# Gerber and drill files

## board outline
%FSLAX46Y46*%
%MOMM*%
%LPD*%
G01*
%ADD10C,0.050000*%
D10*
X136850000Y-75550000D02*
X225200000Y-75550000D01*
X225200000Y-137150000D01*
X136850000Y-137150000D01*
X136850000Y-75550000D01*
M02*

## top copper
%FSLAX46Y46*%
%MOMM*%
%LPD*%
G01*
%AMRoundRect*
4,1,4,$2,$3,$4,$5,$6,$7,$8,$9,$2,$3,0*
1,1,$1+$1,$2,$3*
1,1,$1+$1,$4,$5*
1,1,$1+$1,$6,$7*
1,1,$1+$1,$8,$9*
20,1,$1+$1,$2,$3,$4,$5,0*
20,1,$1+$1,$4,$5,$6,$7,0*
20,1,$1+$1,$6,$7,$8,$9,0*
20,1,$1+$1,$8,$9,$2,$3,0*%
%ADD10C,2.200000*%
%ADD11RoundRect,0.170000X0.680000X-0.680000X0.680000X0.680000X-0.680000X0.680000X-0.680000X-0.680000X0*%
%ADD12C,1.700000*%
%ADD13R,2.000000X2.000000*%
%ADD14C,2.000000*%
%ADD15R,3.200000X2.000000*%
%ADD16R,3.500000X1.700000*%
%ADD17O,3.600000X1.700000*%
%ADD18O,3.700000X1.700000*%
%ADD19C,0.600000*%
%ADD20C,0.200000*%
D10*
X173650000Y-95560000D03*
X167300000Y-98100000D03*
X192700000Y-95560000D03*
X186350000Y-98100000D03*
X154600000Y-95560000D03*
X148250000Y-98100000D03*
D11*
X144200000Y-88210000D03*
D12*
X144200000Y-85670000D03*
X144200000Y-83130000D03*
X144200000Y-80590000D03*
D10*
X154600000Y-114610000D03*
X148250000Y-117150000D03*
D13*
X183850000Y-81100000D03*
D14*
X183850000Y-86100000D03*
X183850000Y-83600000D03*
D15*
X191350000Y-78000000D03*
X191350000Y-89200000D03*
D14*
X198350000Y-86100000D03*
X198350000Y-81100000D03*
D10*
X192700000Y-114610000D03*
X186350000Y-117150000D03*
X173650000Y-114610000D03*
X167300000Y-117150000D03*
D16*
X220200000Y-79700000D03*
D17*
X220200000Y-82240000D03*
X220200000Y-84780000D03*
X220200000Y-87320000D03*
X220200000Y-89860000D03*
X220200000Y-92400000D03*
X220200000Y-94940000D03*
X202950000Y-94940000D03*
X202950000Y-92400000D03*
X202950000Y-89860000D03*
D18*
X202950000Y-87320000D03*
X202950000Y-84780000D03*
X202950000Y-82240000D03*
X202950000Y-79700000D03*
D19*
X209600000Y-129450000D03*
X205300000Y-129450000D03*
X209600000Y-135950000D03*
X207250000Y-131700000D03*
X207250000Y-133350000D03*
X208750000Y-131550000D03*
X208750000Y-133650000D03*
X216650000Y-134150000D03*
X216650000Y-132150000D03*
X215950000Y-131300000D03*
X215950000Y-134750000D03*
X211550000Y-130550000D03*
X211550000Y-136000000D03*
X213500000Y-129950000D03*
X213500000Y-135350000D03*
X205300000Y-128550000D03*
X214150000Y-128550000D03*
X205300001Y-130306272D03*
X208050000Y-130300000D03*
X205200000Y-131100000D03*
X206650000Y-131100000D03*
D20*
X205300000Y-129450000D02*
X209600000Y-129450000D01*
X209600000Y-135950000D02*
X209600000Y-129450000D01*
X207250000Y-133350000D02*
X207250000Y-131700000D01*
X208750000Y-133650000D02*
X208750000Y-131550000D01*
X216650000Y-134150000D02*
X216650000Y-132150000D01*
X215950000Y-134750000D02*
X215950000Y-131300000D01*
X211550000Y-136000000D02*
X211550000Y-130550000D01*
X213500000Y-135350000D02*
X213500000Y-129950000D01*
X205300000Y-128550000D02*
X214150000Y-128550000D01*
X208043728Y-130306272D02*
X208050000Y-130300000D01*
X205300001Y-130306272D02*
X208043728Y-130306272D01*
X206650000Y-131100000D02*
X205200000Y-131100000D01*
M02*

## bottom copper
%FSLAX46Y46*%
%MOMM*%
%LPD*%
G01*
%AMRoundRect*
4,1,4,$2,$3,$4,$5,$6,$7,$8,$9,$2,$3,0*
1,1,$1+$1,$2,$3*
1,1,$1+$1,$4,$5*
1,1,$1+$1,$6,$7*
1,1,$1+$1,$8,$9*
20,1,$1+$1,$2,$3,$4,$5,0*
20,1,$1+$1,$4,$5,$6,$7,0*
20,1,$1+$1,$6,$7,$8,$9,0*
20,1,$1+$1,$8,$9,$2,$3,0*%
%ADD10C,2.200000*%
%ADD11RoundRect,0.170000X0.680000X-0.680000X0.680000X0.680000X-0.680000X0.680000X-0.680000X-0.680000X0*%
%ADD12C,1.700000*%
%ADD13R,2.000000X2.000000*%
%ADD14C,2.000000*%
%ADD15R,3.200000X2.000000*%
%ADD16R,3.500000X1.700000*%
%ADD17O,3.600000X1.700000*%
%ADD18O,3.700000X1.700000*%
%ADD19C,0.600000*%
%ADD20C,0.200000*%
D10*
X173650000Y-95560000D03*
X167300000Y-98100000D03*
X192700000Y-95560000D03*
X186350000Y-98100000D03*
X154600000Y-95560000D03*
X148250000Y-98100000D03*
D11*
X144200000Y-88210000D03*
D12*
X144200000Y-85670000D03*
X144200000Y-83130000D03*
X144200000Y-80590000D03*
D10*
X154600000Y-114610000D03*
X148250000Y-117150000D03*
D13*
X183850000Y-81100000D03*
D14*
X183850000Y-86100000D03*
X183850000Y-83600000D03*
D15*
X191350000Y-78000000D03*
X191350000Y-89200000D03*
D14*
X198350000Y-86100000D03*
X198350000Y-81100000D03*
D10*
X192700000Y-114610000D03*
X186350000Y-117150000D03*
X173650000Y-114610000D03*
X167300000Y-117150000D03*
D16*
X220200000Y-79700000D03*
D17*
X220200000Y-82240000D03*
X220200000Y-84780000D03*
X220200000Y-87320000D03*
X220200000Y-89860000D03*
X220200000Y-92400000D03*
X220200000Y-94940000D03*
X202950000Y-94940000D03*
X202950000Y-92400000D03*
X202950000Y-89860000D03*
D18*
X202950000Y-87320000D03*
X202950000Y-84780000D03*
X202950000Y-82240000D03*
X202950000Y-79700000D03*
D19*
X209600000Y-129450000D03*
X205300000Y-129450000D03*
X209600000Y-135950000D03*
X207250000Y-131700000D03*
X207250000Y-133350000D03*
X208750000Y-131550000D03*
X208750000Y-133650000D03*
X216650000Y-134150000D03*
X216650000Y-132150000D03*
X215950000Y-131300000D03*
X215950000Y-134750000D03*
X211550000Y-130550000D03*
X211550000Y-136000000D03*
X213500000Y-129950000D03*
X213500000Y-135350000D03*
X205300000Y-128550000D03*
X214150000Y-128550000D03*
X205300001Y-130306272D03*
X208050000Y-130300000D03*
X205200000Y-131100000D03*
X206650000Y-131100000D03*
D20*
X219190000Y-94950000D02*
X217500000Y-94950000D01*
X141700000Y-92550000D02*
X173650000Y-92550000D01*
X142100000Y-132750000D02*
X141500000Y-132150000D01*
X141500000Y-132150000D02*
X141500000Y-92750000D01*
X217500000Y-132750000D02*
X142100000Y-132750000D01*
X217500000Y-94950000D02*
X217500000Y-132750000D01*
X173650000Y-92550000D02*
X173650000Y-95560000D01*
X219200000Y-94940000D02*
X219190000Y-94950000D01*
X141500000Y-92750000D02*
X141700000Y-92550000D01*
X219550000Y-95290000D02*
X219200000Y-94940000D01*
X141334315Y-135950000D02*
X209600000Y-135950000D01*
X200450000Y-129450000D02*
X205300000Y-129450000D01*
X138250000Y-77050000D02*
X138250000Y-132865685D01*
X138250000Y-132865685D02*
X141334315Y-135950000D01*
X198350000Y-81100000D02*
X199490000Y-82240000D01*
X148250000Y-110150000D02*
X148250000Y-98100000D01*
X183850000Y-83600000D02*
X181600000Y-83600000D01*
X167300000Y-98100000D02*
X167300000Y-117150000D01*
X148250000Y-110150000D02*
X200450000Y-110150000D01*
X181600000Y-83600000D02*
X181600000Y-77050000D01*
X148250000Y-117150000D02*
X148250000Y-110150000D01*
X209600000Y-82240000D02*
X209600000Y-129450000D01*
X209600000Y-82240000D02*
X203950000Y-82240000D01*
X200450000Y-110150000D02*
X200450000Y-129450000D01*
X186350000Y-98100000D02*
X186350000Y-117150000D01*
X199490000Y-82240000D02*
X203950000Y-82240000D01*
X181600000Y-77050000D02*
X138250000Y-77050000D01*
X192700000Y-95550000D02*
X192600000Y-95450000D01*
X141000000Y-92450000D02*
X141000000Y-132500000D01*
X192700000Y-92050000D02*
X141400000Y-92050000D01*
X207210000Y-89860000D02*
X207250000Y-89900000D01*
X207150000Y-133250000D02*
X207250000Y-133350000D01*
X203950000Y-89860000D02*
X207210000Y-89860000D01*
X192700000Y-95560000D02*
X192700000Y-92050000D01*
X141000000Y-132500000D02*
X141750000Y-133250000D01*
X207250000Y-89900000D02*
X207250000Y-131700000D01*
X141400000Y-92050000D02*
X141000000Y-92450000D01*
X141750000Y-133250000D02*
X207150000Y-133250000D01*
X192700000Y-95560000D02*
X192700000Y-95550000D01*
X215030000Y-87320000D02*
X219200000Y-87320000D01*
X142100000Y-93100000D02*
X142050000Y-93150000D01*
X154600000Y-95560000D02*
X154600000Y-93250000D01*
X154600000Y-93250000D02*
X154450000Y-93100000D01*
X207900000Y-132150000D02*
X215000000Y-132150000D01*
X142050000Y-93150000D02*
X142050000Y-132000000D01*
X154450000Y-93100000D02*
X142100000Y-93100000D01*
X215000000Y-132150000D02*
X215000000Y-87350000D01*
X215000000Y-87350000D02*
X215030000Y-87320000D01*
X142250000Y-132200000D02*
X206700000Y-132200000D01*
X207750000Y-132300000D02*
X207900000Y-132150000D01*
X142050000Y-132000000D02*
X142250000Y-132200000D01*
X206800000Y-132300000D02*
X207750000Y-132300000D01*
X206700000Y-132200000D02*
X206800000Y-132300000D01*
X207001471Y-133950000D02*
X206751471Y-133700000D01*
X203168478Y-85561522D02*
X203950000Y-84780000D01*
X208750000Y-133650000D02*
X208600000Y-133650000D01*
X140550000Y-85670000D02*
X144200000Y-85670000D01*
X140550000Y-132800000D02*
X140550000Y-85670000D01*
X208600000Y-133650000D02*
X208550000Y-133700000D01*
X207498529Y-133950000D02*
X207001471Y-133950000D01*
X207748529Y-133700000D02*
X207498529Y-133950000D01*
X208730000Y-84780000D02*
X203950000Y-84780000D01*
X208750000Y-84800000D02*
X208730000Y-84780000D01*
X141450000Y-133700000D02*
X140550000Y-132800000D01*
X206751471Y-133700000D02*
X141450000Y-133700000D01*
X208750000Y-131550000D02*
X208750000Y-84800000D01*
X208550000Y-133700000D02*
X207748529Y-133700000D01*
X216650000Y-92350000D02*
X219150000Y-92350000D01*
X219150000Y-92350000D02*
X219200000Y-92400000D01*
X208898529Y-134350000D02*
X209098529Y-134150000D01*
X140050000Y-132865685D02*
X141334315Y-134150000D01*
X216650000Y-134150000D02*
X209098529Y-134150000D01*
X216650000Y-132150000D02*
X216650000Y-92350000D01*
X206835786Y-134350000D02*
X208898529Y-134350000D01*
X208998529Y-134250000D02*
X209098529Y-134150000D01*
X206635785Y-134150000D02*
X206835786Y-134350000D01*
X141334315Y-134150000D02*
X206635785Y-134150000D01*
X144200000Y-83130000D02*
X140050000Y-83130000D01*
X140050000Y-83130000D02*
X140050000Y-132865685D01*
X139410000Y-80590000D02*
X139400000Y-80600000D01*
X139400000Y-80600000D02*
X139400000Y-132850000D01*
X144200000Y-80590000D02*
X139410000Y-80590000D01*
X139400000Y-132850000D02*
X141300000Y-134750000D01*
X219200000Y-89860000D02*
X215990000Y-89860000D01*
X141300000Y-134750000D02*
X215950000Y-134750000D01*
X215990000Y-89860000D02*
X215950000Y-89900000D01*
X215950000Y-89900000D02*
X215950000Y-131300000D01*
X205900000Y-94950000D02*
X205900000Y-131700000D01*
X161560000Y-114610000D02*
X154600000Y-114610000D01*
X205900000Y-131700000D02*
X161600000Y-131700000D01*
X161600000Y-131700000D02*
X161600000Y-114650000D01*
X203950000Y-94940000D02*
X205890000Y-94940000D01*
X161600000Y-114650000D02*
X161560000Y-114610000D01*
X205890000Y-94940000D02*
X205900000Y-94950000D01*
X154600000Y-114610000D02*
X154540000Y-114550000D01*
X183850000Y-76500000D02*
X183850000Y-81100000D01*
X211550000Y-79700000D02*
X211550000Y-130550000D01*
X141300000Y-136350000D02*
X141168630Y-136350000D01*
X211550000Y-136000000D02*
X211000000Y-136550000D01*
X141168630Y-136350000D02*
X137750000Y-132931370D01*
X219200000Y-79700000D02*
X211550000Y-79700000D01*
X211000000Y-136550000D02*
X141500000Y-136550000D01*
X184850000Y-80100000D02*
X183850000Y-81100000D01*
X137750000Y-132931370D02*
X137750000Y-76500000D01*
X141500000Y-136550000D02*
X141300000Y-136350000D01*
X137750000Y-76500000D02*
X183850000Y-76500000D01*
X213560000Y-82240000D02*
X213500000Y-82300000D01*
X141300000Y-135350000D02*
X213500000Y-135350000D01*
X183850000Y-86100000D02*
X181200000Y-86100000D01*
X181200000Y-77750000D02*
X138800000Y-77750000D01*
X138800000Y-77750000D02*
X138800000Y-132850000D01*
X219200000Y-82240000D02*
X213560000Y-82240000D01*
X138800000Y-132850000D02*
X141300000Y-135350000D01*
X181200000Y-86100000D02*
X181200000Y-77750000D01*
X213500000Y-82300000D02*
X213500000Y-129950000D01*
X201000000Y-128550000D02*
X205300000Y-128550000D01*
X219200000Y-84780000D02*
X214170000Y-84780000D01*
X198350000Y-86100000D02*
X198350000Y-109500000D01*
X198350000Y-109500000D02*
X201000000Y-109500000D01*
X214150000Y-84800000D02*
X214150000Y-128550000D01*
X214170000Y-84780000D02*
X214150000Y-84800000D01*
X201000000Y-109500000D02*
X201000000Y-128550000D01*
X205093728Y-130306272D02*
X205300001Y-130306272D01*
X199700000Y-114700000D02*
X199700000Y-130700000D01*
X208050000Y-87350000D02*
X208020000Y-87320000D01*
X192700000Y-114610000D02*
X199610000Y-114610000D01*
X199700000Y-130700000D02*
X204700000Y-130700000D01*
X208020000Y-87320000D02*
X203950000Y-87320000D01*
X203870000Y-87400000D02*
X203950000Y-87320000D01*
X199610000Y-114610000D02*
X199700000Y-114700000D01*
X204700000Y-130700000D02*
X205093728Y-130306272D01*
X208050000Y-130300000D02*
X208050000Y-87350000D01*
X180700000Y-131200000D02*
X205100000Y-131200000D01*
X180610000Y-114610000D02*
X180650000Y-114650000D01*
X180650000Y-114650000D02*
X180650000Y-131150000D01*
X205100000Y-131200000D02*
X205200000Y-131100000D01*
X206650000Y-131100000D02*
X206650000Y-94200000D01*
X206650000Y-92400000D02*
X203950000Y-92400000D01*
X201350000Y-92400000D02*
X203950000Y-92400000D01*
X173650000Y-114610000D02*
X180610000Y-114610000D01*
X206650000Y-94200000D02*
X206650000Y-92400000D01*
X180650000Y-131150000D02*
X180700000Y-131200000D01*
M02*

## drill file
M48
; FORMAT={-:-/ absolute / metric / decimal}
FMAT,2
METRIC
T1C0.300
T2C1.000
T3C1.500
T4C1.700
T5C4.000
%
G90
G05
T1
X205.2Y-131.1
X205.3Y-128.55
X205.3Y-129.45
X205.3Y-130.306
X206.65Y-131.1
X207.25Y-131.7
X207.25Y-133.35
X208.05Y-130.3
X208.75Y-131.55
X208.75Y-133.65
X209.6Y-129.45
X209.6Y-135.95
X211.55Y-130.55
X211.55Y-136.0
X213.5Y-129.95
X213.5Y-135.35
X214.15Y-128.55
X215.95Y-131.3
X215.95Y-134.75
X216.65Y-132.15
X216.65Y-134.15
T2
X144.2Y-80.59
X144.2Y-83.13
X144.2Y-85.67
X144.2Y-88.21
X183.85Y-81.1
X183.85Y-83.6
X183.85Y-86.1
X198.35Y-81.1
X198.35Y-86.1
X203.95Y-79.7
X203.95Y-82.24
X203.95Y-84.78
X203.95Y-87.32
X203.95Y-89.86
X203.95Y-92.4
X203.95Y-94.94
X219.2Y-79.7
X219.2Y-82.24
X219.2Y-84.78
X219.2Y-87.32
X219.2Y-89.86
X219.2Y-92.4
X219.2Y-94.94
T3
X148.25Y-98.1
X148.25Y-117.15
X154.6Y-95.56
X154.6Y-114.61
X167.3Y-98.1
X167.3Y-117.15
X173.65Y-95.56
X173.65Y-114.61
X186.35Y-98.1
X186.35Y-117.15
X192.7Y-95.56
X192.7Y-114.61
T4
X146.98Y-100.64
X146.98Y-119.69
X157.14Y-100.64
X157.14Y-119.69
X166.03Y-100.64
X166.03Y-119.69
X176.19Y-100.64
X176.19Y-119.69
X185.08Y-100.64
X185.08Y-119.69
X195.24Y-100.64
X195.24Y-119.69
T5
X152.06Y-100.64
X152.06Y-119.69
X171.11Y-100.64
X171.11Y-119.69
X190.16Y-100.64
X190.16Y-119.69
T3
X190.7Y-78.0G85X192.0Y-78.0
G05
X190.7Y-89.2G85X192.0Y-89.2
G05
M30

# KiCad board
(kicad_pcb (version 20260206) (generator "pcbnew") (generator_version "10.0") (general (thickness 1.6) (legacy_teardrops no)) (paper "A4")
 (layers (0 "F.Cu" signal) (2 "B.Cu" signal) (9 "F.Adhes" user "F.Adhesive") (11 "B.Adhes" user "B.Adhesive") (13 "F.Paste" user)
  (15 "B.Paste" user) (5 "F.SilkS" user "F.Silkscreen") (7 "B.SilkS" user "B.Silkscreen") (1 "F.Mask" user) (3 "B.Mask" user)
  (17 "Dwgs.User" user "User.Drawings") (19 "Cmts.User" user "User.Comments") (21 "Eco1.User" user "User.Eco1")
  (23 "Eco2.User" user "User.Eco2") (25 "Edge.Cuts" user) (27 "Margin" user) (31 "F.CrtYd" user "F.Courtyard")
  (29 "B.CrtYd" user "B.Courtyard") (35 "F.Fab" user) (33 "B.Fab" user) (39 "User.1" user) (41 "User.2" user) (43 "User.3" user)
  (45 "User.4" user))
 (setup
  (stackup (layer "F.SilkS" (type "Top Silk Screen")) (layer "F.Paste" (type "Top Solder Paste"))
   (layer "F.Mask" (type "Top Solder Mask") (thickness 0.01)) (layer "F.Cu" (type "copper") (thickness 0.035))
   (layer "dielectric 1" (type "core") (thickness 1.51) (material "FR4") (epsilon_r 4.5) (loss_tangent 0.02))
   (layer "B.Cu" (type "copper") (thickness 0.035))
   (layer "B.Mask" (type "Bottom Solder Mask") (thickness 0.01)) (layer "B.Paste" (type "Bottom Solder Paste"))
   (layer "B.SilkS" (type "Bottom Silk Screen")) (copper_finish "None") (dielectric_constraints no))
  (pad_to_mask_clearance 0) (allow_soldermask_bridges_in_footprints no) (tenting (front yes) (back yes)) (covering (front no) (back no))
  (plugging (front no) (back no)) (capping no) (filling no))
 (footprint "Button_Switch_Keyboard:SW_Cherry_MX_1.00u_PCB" (layer "F.Cu") (at 173.65 95.56)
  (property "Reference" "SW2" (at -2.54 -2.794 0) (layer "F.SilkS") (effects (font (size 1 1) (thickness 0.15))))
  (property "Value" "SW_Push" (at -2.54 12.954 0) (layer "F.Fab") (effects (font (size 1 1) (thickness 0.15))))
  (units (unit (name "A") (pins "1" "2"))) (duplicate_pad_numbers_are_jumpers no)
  (pad "" np_thru_hole circle (at -7.62 5.08) (size 1.7 1.7) (drill 1.7) (layers "*.Cu" "*.Mask"))
  (pad "" np_thru_hole circle (at -2.54 5.08) (size 4 4) (drill 4) (layers "*.Cu" "*.Mask"))
  (pad "" np_thru_hole circle (at 2.54 5.08) (size 1.7 1.7) (drill 1.7) (layers "*.Cu" "*.Mask"))
  (pad "1" thru_hole circle (at 0 0) (size 2.2 2.2) (drill 1.5) (layers "*.Cu" "*.Mask") (remove_unused_layers no)
   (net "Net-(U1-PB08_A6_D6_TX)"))
  (pad "2" thru_hole circle (at -6.35 2.54) (size 2.2 2.2) (drill 1.5) (layers "*.Cu" "*.Mask") (remove_unused_layers no) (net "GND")))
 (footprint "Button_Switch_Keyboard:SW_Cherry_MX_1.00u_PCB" (layer "F.Cu") (at 192.7 95.56)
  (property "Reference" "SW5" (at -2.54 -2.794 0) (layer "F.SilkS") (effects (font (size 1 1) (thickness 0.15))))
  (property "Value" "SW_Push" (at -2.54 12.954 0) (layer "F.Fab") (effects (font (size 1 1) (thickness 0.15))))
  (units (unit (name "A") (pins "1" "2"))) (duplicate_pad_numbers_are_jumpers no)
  (pad "" np_thru_hole circle (at -7.62 5.08) (size 1.7 1.7) (drill 1.7) (layers "*.Cu" "*.Mask"))
  (pad "" np_thru_hole circle (at -2.54 5.08) (size 4 4) (drill 4) (layers "*.Cu" "*.Mask"))
  (pad "" np_thru_hole circle (at 2.54 5.08) (size 1.7 1.7) (drill 1.7) (layers "*.Cu" "*.Mask"))
  (pad "1" thru_hole circle (at 0 0) (size 2.2 2.2) (drill 1.5) (layers "*.Cu" "*.Mask") (remove_unused_layers no)
   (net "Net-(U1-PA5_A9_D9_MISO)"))
  (pad "2" thru_hole circle (at -6.35 2.54) (size 2.2 2.2) (drill 1.5) (layers "*.Cu" "*.Mask") (remove_unused_layers no) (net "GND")))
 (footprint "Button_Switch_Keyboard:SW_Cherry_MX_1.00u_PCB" (layer "F.Cu") (at 154.6 95.56)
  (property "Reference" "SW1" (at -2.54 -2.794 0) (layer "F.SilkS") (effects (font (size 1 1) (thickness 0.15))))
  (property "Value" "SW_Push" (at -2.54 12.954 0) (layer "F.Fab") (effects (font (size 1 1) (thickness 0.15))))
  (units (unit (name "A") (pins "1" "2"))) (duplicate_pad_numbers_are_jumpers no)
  (pad "" np_thru_hole circle (at -7.62 5.08) (size 1.7 1.7) (drill 1.7) (layers "*.Cu" "*.Mask"))
  (pad "" np_thru_hole circle (at -2.54 5.08) (size 4 4) (drill 4) (layers "*.Cu" "*.Mask"))
  (pad "" np_thru_hole circle (at 2.54 5.08) (size 1.7 1.7) (drill 1.7) (layers "*.Cu" "*.Mask"))
  (pad "1" thru_hole circle (at 0 0) (size 2.2 2.2) (drill 1.5) (layers "*.Cu" "*.Mask") (remove_unused_layers no)
   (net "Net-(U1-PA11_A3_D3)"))
  (pad "2" thru_hole circle (at -6.35 2.54) (size 2.2 2.2) (drill 1.5) (layers "*.Cu" "*.Mask") (remove_unused_layers no) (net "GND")))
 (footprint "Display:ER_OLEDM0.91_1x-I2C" (layer "F.Cu") (at 144.2 88.21 90)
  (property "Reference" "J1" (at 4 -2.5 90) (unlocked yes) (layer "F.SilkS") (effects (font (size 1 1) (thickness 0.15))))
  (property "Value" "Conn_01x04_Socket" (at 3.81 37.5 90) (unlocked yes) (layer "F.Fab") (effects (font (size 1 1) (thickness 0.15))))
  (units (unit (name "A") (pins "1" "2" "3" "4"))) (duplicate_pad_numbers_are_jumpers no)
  (pad "1" thru_hole roundrect (at 0 0 90) (size 1.7 1.7) (drill 1) (layers "*.Cu" "*.Mask") (remove_unused_layers no)
   (roundrect_rratio 0.1) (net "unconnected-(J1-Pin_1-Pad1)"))
  (pad "2" thru_hole circle (at 2.54 0 90) (size 1.7 1.7) (drill 1) (layers "*.Cu" "*.Mask") (remove_unused_layers no)
   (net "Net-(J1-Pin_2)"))
  (pad "3" thru_hole circle (at 5.08 0 90) (size 1.7 1.7) (drill 1) (layers "*.Cu" "*.Mask") (remove_unused_layers no)
   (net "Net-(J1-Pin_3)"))
  (pad "4" thru_hole circle (at 7.62 0 90) (size 1.7 1.7) (drill 1) (layers "*.Cu" "*.Mask") (remove_unused_layers no)
   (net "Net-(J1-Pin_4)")))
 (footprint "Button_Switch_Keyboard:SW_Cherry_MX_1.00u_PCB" (layer "F.Cu") (at 154.6 114.61)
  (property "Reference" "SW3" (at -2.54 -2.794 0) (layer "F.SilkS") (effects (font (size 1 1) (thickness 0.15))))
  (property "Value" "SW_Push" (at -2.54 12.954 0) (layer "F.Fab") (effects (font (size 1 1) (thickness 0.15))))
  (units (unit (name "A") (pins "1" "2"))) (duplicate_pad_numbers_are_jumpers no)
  (pad "" np_thru_hole circle (at -7.62 5.08) (size 1.7 1.7) (drill 1.7) (layers "*.Cu" "*.Mask"))
  (pad "" np_thru_hole circle (at -2.54 5.08) (size 4 4) (drill 4) (layers "*.Cu" "*.Mask"))
  (pad "" np_thru_hole circle (at 2.54 5.08) (size 1.7 1.7) (drill 1.7) (layers "*.Cu" "*.Mask"))
  (pad "1" thru_hole circle (at 0 0) (size 2.2 2.2) (drill 1.5) (layers "*.Cu" "*.Mask") (remove_unused_layers no)
   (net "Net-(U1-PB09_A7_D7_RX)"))
  (pad "2" thru_hole circle (at -6.35 2.54) (size 2.2 2.2) (drill 1.5) (layers "*.Cu" "*.Mask") (remove_unused_layers no) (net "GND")))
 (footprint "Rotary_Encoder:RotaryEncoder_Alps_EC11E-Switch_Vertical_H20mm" (layer "F.Cu") (at 183.85 81.1)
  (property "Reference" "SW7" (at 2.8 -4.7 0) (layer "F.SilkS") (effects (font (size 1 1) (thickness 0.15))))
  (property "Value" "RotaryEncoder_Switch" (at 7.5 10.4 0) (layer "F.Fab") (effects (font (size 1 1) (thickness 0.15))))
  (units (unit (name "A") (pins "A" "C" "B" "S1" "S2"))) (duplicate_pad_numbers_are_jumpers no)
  (pad "A" thru_hole rect (at 0 0) (size 2 2) (drill 1) (layers "*.Cu" "*.Mask") (remove_unused_layers no) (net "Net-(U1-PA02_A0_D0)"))
  (pad "B" thru_hole circle (at 0 5) (size 2 2) (drill 1) (layers "*.Cu" "*.Mask") (remove_unused_layers no) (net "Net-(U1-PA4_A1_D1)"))
  (pad "C" thru_hole circle (at 0 2.5) (size 2 2) (drill 1) (layers "*.Cu" "*.Mask") (remove_unused_layers no) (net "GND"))
  (pad "MP" thru_hole rect (at 7.5 -3.1) (size 3.2 2) (drill oval 2.8 1.5) (layers "*.Cu" "*.Mask") (remove_unused_layers no))
  (pad "MP" thru_hole rect (at 7.5 8.1) (size 3.2 2) (drill oval 2.8 1.5) (layers "*.Cu" "*.Mask") (remove_unused_layers no))
  (pad "S1" thru_hole circle (at 14.5 5) (size 2 2) (drill 1) (layers "*.Cu" "*.Mask") (remove_unused_layers no) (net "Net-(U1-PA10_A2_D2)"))
  (pad "S2" thru_hole circle (at 14.5 0) (size 2 2) (drill 1) (layers "*.Cu" "*.Mask") (remove_unused_layers no) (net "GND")))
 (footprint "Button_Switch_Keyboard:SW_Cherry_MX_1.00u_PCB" (layer "F.Cu") (at 192.7 114.61)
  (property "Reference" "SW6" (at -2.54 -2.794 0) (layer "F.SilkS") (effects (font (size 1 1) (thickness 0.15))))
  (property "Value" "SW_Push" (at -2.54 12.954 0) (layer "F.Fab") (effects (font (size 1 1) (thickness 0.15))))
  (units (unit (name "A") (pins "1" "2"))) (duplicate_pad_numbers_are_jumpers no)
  (pad "" np_thru_hole circle (at -7.62 5.08) (size 1.7 1.7) (drill 1.7) (layers "*.Cu" "*.Mask"))
  (pad "" np_thru_hole circle (at -2.54 5.08) (size 4 4) (drill 4) (layers "*.Cu" "*.Mask"))
  (pad "" np_thru_hole circle (at 2.54 5.08) (size 1.7 1.7) (drill 1.7) (layers "*.Cu" "*.Mask"))
  (pad "1" thru_hole circle (at 0 0) (size 2.2 2.2) (drill 1.5) (layers "*.Cu" "*.Mask") (remove_unused_layers no)
   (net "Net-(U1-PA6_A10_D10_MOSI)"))
  (pad "2" thru_hole circle (at -6.35 2.54) (size 2.2 2.2) (drill 1.5) (layers "*.Cu" "*.Mask") (remove_unused_layers no) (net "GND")))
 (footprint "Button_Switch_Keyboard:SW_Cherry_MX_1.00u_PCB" (layer "F.Cu") (at 173.65 114.61)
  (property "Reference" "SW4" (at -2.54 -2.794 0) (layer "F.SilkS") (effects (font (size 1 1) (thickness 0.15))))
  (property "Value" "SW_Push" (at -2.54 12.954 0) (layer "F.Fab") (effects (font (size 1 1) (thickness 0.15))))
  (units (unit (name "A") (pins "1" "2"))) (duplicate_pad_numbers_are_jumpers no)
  (pad "" np_thru_hole circle (at -7.62 5.08) (size 1.7 1.7) (drill 1.7) (layers "*.Cu" "*.Mask"))
  (pad "" np_thru_hole circle (at -2.54 5.08) (size 4 4) (drill 4) (layers "*.Cu" "*.Mask"))
  (pad "" np_thru_hole circle (at 2.54 5.08) (size 1.7 1.7) (drill 1.7) (layers "*.Cu" "*.Mask"))
  (pad "1" thru_hole circle (at 0 0) (size 2.2 2.2) (drill 1.5) (layers "*.Cu" "*.Mask") (remove_unused_layers no)
   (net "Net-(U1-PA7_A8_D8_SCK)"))
  (pad "2" thru_hole circle (at -6.35 2.54) (size 2.2 2.2) (drill 1.5) (layers "*.Cu" "*.Mask") (remove_unused_layers no) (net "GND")))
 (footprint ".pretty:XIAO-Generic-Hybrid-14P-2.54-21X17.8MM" (layer "B.Cu") (at 211.575 87.32 180)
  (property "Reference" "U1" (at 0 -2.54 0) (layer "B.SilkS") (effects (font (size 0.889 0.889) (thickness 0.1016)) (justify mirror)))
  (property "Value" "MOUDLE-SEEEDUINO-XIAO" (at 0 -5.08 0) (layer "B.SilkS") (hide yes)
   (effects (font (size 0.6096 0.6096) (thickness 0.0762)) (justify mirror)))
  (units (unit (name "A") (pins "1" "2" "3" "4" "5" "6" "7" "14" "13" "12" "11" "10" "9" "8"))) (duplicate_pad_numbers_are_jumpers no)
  (pad "1" thru_hole rect (at -7.625 7.62 180) (size 3.5 1.7) (drill 1 (offset -1 0)) (layers "*.Cu" "*.Mask") (remove_unused_layers no)
   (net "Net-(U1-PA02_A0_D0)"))
  (pad "2" thru_hole oval (at -7.625 5.08 180) (size 3.6 1.7) (drill 1 (offset -1 0)) (layers "*.Cu" "*.Mask") (remove_unused_layers no)
   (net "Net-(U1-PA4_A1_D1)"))
  (pad "3" thru_hole oval (at -7.625 2.54 180) (size 3.6 1.7) (drill 1 (offset -1 0)) (layers "*.Cu" "*.Mask") (remove_unused_layers no)
   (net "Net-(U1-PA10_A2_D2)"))
  (pad "4" thru_hole oval (at -7.625 0 180) (size 3.6 1.7) (drill 1 (offset -1 0)) (layers "*.Cu" "*.Mask") (remove_unused_layers no)
   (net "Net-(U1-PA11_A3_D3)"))
  (pad "5" thru_hole oval (at -7.625 -2.54 180) (size 3.6 1.7) (drill 1 (offset -1 0)) (layers "*.Cu" "*.Mask") (remove_unused_layers no)
   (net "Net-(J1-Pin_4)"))
  (pad "6" thru_hole oval (at -7.625 -5.08) (size 3.6 1.7) (drill 1 (offset 1 0)) (layers "*.Cu" "*.Mask") (remove_unused_layers no)
   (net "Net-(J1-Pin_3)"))
  (pad "7" thru_hole oval (at -7.625 -7.62 180) (size 3.6 1.7) (drill 1 (offset -1 0)) (layers "*.Cu" "*.Mask") (remove_unused_layers no)
   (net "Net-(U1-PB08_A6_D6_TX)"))
  (pad "8" thru_hole oval (at 7.625 -7.62 180) (size 3.6 1.7) (drill 1 (offset 1 0)) (layers "*.Cu" "*.Mask") (remove_unused_layers no)
   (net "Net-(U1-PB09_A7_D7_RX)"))
  (pad "9" thru_hole oval (at 7.625 -5.08 180) (size 3.6 1.7) (drill 1 (offset 1 0)) (layers "*.Cu" "*.Mask") (remove_unused_layers no)
   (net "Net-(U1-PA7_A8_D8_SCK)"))
  (pad "10" thru_hole oval (at 7.625 -2.54 180) (size 3.6 1.7) (drill 1 (offset 1 0)) (layers "*.Cu" "*.Mask") (remove_unused_layers no)
   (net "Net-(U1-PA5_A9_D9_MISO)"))
  (pad "11" thru_hole oval (at 7.625 0 180) (size 3.7 1.7) (drill 1 (offset 1 0)) (layers "*.Cu" "*.Mask") (remove_unused_layers no)
   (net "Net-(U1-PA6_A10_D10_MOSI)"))
  (pad "12" thru_hole oval (at 7.625 2.54 180) (size 3.7 1.7) (drill 1 (offset 1 0)) (layers "*.Cu" "*.Mask") (remove_unused_layers no)
   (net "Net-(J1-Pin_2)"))
  (pad "13" thru_hole oval (at 7.625 5.08 180) (size 3.7 1.7) (drill 1 (offset 1 0)) (layers "*.Cu" "*.Mask") (remove_unused_layers no)
   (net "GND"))
  (pad "14" thru_hole oval (at 7.625 7.62 180) (size 3.7 1.7) (drill 1 (offset 1 0)) (layers "*.Cu" "*.Mask") (remove_unused_layers no)
   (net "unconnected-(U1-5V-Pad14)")))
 (gr_rect (start 136.85 75.55) (end 225.2 137.15) (stroke (width 0.05) (type default)) (fill no) (layer "Edge.Cuts"))
 (segment (start 219.19 94.95) (end 217.5 94.95) (width 0.2) (layer "B.Cu") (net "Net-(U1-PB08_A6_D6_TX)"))
 (segment (start 141.7 92.55) (end 173.65 92.55) (width 0.2) (layer "B.Cu") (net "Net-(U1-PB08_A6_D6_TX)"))
 (segment (start 142.1 132.75) (end 141.5 132.15) (width 0.2) (layer "B.Cu") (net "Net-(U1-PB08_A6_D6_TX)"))
 (segment (start 141.5 132.15) (end 141.5 92.75) (width 0.2) (layer "B.Cu") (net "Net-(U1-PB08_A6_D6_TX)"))
 (segment (start 217.5 132.75) (end 142.1 132.75) (width 0.2) (layer "B.Cu") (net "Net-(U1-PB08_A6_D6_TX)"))
 (segment (start 217.5 94.95) (end 217.5 132.75) (width 0.2) (layer "B.Cu") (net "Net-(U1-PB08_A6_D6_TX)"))
 (segment (start 173.65 92.55) (end 173.65 95.56) (width 0.2) (layer "B.Cu") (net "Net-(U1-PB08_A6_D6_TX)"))
 (segment (start 219.2 94.94) (end 219.19 94.95) (width 0.2) (layer "B.Cu") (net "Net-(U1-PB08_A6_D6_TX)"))
 (segment (start 141.5 92.75) (end 141.7 92.55) (width 0.2) (layer "B.Cu") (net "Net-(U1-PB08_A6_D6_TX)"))
 (segment (start 219.55 95.29) (end 219.2 94.94) (width 0.2) (layer "B.Cu") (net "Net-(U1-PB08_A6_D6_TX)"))
 (segment (start 205.3 129.45) (end 209.6 129.45) (width 0.2) (layer "F.Cu") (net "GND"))
 (segment (start 209.6 135.95) (end 209.6 129.45) (width 0.2) (layer "F.Cu") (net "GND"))
 (via (at 209.6 129.45) (size 0.6) (drill 0.3) (layers "F.Cu" "B.Cu") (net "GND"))
 (via (at 205.3 129.45) (size 0.6) (drill 0.3) (layers "F.Cu" "B.Cu") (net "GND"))
 (via (at 209.6 135.95) (size 0.6) (drill 0.3) (layers "F.Cu" "B.Cu") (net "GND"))
 (segment (start 141.334315 135.95) (end 209.6 135.95) (width 0.2) (layer "B.Cu") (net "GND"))
 (segment (start 200.45 129.45) (end 205.3 129.45) (width 0.2) (layer "B.Cu") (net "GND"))
 (segment (start 138.25 77.05) (end 138.25 132.865685) (width 0.2) (layer "B.Cu") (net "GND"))
 (segment (start 138.25 132.865685) (end 141.334315 135.95) (width 0.2) (layer "B.Cu") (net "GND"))
 (segment (start 198.35 81.1) (end 199.49 82.24) (width 0.2) (layer "B.Cu") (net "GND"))
 (segment (start 148.25 110.15) (end 148.25 98.1) (width 0.2) (layer "B.Cu") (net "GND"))
 (segment (start 183.85 83.6) (end 181.6 83.6) (width 0.2) (layer "B.Cu") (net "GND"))
 (segment (start 167.3 98.1) (end 167.3 117.15) (width 0.2) (layer "B.Cu") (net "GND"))
 (segment (start 148.25 110.15) (end 200.45 110.15) (width 0.2) (layer "B.Cu") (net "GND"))
 (segment (start 181.6 83.6) (end 181.6 77.05) (width 0.2) (layer "B.Cu") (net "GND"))
 (segment (start 148.25 117.15) (end 148.25 110.15) (width 0.2) (layer "B.Cu") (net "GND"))
 (segment (start 209.6 82.24) (end 209.6 129.45) (width 0.2) (layer "B.Cu") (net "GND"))
 (segment (start 209.6 82.24) (end 203.95 82.24) (width 0.2) (layer "B.Cu") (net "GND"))
 (segment (start 200.45 110.15) (end 200.45 129.45) (width 0.2) (layer "B.Cu") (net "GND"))
 (segment (start 186.35 98.1) (end 186.35 117.15) (width 0.2) (layer "B.Cu") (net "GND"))
 (segment (start 199.49 82.24) (end 203.95 82.24) (width 0.2) (layer "B.Cu") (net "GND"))
 (segment (start 181.6 77.05) (end 138.25 77.05) (width 0.2) (layer "B.Cu") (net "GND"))
 (segment (start 207.25 133.35) (end 207.25 131.7) (width 0.2) (layer "F.Cu") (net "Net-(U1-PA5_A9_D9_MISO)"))
 (via (at 207.25 131.7) (size 0.6) (drill 0.3) (layers "F.Cu" "B.Cu") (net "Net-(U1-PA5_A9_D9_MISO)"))
 (via (at 207.25 133.35) (size 0.6) (drill 0.3) (layers "F.Cu" "B.Cu") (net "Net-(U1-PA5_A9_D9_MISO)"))
 (segment (start 192.7 95.55) (end 192.6 95.45) (width 0.2) (layer "B.Cu") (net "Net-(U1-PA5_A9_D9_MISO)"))
 (segment (start 141 92.45) (end 141 132.5) (width 0.2) (layer "B.Cu") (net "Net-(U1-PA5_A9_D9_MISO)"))
 (segment (start 192.7 92.05) (end 141.4 92.05) (width 0.2) (layer "B.Cu") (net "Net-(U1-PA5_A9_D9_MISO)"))
 (segment (start 207.21 89.86) (end 207.25 89.9) (width 0.2) (layer "B.Cu") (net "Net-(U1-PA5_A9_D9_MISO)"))
 (segment (start 207.15 133.25) (end 207.25 133.35) (width 0.2) (layer "B.Cu") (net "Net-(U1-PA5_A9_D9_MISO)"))
 (segment (start 203.95 89.86) (end 207.21 89.86) (width 0.2) (layer "B.Cu") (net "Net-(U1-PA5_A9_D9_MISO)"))
 (segment (start 192.7 95.56) (end 192.7 92.05) (width 0.2) (layer "B.Cu") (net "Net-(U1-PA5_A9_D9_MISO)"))
 (segment (start 141 132.5) (end 141.75 133.25) (width 0.2) (layer "B.Cu") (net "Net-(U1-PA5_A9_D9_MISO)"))
 (segment (start 207.25 89.9) (end 207.25 131.7) (width 0.2) (layer "B.Cu") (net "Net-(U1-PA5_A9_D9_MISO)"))
 (segment (start 141.4 92.05) (end 141 92.45) (width 0.2) (layer "B.Cu") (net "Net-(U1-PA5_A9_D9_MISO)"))
 (segment (start 141.75 133.25) (end 207.15 133.25) (width 0.2) (layer "B.Cu") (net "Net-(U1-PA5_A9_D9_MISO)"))
 (segment (start 192.7 95.56) (end 192.7 95.55) (width 0.2) (layer "B.Cu") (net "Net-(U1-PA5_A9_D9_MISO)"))
 (segment (start 215.03 87.32) (end 219.2 87.32) (width 0.2) (layer "B.Cu") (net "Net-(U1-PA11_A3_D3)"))
 (segment (start 142.1 93.1) (end 142.05 93.15) (width 0.2) (layer "B.Cu") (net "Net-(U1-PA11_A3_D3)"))
 (segment (start 154.6 95.56) (end 154.6 93.25) (width 0.2) (layer "B.Cu") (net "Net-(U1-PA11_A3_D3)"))
 (segment (start 154.6 93.25) (end 154.45 93.1) (width 0.2) (layer "B.Cu") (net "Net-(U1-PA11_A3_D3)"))
 (segment (start 207.9 132.15) (end 215 132.15) (width 0.2) (layer "B.Cu") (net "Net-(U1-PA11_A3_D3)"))
 (segment (start 142.05 93.15) (end 142.05 132) (width 0.2) (layer "B.Cu") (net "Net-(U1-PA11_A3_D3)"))
 (segment (start 154.45 93.1) (end 142.1 93.1) (width 0.2) (layer "B.Cu") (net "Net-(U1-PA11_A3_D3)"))
 (segment (start 215 132.15) (end 215 87.35) (width 0.2) (layer "B.Cu") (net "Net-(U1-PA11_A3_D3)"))
 (segment (start 215 87.35) (end 215.03 87.32) (width 0.2) (layer "B.Cu") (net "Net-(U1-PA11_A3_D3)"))
 (segment (start 142.25 132.2) (end 206.7 132.2) (width 0.2) (layer "B.Cu") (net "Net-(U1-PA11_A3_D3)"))
 (segment (start 207.75 132.3) (end 207.9 132.15) (width 0.2) (layer "B.Cu") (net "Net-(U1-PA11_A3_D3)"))
 (segment (start 142.05 132) (end 142.25 132.2) (width 0.2) (layer "B.Cu") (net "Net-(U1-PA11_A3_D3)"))
 (segment (start 206.8 132.3) (end 207.75 132.3) (width 0.2) (layer "B.Cu") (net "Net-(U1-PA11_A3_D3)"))
 (segment (start 206.7 132.2) (end 206.8 132.3) (width 0.2) (layer "B.Cu") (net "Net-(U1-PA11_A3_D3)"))
 (segment (start 208.75 133.65) (end 208.75 131.55) (width 0.2) (layer "F.Cu") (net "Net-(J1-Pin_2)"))
 (via (at 208.75 131.55) (size 0.6) (drill 0.3) (layers "F.Cu" "B.Cu") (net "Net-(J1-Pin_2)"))
 (via (at 208.75 133.65) (size 0.6) (drill 0.3) (layers "F.Cu" "B.Cu") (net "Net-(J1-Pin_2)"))
 (segment (start 207.001471 133.95) (end 206.751471 133.7) (width 0.2) (layer "B.Cu") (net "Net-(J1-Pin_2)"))
 (segment (start 203.168478 85.561522) (end 203.95 84.78) (width 0.2) (layer "B.Cu") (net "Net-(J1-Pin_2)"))
 (segment (start 208.75 133.65) (end 208.6 133.65) (width 0.2) (layer "B.Cu") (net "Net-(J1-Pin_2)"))
 (segment (start 140.55 85.67) (end 144.2 85.67) (width 0.2) (layer "B.Cu") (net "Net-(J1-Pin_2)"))
 (segment (start 140.55 132.8) (end 140.55 85.67) (width 0.2) (layer "B.Cu") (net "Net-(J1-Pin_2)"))
 (segment (start 208.6 133.65) (end 208.55 133.7) (width 0.2) (layer "B.Cu") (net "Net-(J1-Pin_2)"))
 (segment (start 207.498529 133.95) (end 207.001471 133.95) (width 0.2) (layer "B.Cu") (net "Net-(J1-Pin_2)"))
 (segment (start 207.748529 133.7) (end 207.498529 133.95) (width 0.2) (layer "B.Cu") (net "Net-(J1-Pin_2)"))
 (segment (start 208.73 84.78) (end 203.95 84.78) (width 0.2) (layer "B.Cu") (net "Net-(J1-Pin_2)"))
 (segment (start 208.75 84.8) (end 208.73 84.78) (width 0.2) (layer "B.Cu") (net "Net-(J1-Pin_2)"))
 (segment (start 141.45 133.7) (end 140.55 132.8) (width 0.2) (layer "B.Cu") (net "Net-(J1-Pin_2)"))
 (segment (start 206.751471 133.7) (end 141.45 133.7) (width 0.2) (layer "B.Cu") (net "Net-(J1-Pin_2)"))
 (segment (start 208.75 131.55) (end 208.75 84.8) (width 0.2) (layer "B.Cu") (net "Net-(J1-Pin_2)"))
 (segment (start 208.55 133.7) (end 207.748529 133.7) (width 0.2) (layer "B.Cu") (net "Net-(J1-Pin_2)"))
 (segment (start 216.65 134.15) (end 216.65 132.15) (width 0.2) (layer "F.Cu") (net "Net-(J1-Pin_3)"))
 (via (at 216.65 134.15) (size 0.6) (drill 0.3) (layers "F.Cu" "B.Cu") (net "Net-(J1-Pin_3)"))
 (via (at 216.65 132.15) (size 0.6) (drill 0.3) (layers "F.Cu" "B.Cu") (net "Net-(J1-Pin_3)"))
 (segment (start 216.65 92.35) (end 219.15 92.35) (width 0.2) (layer "B.Cu") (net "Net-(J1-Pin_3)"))
 (segment (start 219.15 92.35) (end 219.2 92.4) (width 0.2) (layer "B.Cu") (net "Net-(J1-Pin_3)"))
 (segment (start 208.898529 134.35) (end 209.098529 134.15) (width 0.2) (layer "B.Cu") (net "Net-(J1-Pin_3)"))
 (segment (start 140.05 132.865685) (end 141.334315 134.15) (width 0.2) (layer "B.Cu") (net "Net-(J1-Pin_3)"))
 (segment (start 216.65 134.15) (end 209.098529 134.15) (width 0.2) (layer "B.Cu") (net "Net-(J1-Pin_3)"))
 (segment (start 216.65 132.15) (end 216.65 92.35) (width 0.2) (layer "B.Cu") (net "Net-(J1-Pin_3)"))
 (segment (start 206.835786 134.35) (end 208.898529 134.35) (width 0.2) (layer "B.Cu") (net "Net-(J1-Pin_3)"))
 (segment (start 208.998529 134.25) (end 209.098529 134.15) (width 0.2) (layer "B.Cu") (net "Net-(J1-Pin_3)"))
 (segment (start 206.635785 134.15) (end 206.835786 134.35) (width 0.2) (layer "B.Cu") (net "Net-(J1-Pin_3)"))
 (segment (start 141.334315 134.15) (end 206.635785 134.15) (width 0.2) (layer "B.Cu") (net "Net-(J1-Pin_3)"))
 (segment (start 144.2 83.13) (end 140.05 83.13) (width 0.2) (layer "B.Cu") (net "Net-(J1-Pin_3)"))
 (segment (start 140.05 83.13) (end 140.05 132.865685) (width 0.2) (layer "B.Cu") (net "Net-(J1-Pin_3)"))
 (segment (start 215.95 134.75) (end 215.95 131.3) (width 0.2) (layer "F.Cu") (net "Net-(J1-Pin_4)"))
 (via (at 215.95 131.3) (size 0.6) (drill 0.3) (layers "F.Cu" "B.Cu") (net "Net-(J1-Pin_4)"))
 (via (at 215.95 134.75) (size 0.6) (drill 0.3) (layers "F.Cu" "B.Cu") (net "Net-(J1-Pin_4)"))
 (segment (start 139.41 80.59) (end 139.4 80.6) (width 0.2) (layer "B.Cu") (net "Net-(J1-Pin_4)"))
 (segment (start 139.4 80.6) (end 139.4 132.85) (width 0.2) (layer "B.Cu") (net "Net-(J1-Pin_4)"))
 (segment (start 144.2 80.59) (end 139.41 80.59) (width 0.2) (layer "B.Cu") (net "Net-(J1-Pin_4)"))
 (segment (start 139.4 132.85) (end 141.3 134.75) (width 0.2) (layer "B.Cu") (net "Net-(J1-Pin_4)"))
 (segment (start 219.2 89.86) (end 215.99 89.86) (width 0.2) (layer "B.Cu") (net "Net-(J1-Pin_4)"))
 (segment (start 141.3 134.75) (end 215.95 134.75) (width 0.2) (layer "B.Cu") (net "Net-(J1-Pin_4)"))
 (segment (start 215.99 89.86) (end 215.95 89.9) (width 0.2) (layer "B.Cu") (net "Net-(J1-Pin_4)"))
 (segment (start 215.95 89.9) (end 215.95 131.3) (width 0.2) (layer "B.Cu") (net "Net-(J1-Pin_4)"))
 (segment (start 205.9 94.95) (end 205.9 131.7) (width 0.2) (layer "B.Cu") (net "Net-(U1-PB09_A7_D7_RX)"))
 (segment (start 161.56 114.61) (end 154.6 114.61) (width 0.2) (layer "B.Cu") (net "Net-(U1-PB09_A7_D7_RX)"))
 (segment (start 205.9 131.7) (end 161.6 131.7) (width 0.2) (layer "B.Cu") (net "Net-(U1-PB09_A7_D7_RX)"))
 (segment (start 161.6 131.7) (end 161.6 114.65) (width 0.2) (layer "B.Cu") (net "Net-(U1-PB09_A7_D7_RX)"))
 (segment (start 203.95 94.94) (end 205.89 94.94) (width 0.2) (layer "B.Cu") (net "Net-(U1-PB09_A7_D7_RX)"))
 (segment (start 161.6 114.65) (end 161.56 114.61) (width 0.2) (layer "B.Cu") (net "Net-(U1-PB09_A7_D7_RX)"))
 (segment (start 205.89 94.94) (end 205.9 94.95) (width 0.2) (layer "B.Cu") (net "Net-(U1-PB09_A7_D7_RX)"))
 (segment (start 154.6 114.61) (end 154.54 114.55) (width 0.2) (layer "B.Cu") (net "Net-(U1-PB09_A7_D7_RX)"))
 (segment (start 211.55 136) (end 211.55 130.55) (width 0.2) (layer "F.Cu") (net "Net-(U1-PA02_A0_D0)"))
 (via (at 211.55 130.55) (size 0.6) (drill 0.3) (layers "F.Cu" "B.Cu") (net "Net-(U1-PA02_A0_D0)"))
 (via (at 211.55 136) (size 0.6) (drill 0.3) (layers "F.Cu" "B.Cu") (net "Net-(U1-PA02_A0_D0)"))
 (segment (start 183.85 76.5) (end 183.85 81.1) (width 0.2) (layer "B.Cu") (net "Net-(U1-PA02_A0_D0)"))
 (segment (start 211.55 79.7) (end 211.55 130.55) (width 0.2) (layer "B.Cu") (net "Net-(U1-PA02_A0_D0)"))
 (segment (start 141.3 136.35) (end 141.16863 136.35) (width 0.2) (layer "B.Cu") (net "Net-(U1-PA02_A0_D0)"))
 (segment (start 211.55 136) (end 211 136.55) (width 0.2) (layer "B.Cu") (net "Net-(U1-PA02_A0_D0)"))
 (segment (start 141.16863 136.35) (end 137.75 132.93137) (width 0.2) (layer "B.Cu") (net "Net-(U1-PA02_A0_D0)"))
 (segment (start 219.2 79.7) (end 211.55 79.7) (width 0.2) (layer "B.Cu") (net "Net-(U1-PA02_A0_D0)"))
 (segment (start 211 136.55) (end 141.5 136.55) (width 0.2) (layer "B.Cu") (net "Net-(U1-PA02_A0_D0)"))
 (segment (start 184.85 80.1) (end 183.85 81.1) (width 0.2) (layer "B.Cu") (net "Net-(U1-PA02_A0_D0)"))
 (segment (start 137.75 132.93137) (end 137.75 76.5) (width 0.2) (layer "B.Cu") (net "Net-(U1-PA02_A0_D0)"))
 (segment (start 141.5 136.55) (end 141.3 136.35) (width 0.2) (layer "B.Cu") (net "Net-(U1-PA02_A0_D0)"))
 (segment (start 137.75 76.5) (end 183.85 76.5) (width 0.2) (layer "B.Cu") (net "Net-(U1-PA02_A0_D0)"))
 (segment (start 213.5 135.35) (end 213.5 129.95) (width 0.2) (layer "F.Cu") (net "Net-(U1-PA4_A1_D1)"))
 (via (at 213.5 129.95) (size 0.6) (drill 0.3) (layers "F.Cu" "B.Cu") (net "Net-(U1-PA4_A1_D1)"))
 (via (at 213.5 135.35) (size 0.6) (drill 0.3) (layers "F.Cu" "B.Cu") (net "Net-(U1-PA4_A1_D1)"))
 (segment (start 213.56 82.24) (end 213.5 82.3) (width 0.2) (layer "B.Cu") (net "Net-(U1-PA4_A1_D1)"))
 (segment (start 141.3 135.35) (end 213.5 135.35) (width 0.2) (layer "B.Cu") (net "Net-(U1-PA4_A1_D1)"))
 (segment (start 183.85 86.1) (end 181.2 86.1) (width 0.2) (layer "B.Cu") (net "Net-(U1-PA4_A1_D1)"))
 (segment (start 181.2 77.75) (end 138.8 77.75) (width 0.2) (layer "B.Cu") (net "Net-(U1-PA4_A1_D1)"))
 (segment (start 138.8 77.75) (end 138.8 132.85) (width 0.2) (layer "B.Cu") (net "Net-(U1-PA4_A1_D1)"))
 (segment (start 219.2 82.24) (end 213.56 82.24) (width 0.2) (layer "B.Cu") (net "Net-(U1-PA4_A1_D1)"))
 (segment (start 138.8 132.85) (end 141.3 135.35) (width 0.2) (layer "B.Cu") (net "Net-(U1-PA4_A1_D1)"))
 (segment (start 181.2 86.1) (end 181.2 77.75) (width 0.2) (layer "B.Cu") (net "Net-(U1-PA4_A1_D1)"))
 (segment (start 213.5 82.3) (end 213.5 129.95) (width 0.2) (layer "B.Cu") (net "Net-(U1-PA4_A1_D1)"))
 (segment (start 205.3 128.55) (end 214.15 128.55) (width 0.2) (layer "F.Cu") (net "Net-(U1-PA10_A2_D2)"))
 (via (at 205.3 128.55) (size 0.6) (drill 0.3) (layers "F.Cu" "B.Cu") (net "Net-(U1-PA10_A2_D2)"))
 (via (at 214.15 128.55) (size 0.6) (drill 0.3) (layers "F.Cu" "B.Cu") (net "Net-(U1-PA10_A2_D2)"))
 (segment (start 201 128.55) (end 205.3 128.55) (width 0.2) (layer "B.Cu") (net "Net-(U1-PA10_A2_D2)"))
 (segment (start 219.2 84.78) (end 214.17 84.78) (width 0.2) (layer "B.Cu") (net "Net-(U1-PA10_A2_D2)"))
 (segment (start 198.35 86.1) (end 198.35 109.5) (width 0.2) (layer "B.Cu") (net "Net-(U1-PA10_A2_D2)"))
 (segment (start 198.35 109.5) (end 201 109.5) (width 0.2) (layer "B.Cu") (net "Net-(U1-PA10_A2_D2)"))
 (segment (start 214.15 84.8) (end 214.15 128.55) (width 0.2) (layer "B.Cu") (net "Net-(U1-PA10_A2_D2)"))
 (segment (start 214.17 84.78) (end 214.15 84.8) (width 0.2) (layer "B.Cu") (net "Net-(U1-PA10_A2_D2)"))
 (segment (start 201 109.5) (end 201 128.55) (width 0.2) (layer "B.Cu") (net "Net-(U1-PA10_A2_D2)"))
 (segment (start 208.043728 130.306272) (end 208.05 130.3) (width 0.2) (layer "F.Cu") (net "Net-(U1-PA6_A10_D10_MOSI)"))
 (segment (start 205.300001 130.306272) (end 208.043728 130.306272) (width 0.2) (layer "F.Cu") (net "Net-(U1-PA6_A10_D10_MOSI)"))
 (via (at 205.300001 130.306272) (size 0.6) (drill 0.3) (layers "F.Cu" "B.Cu") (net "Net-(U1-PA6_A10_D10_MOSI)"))
 (via (at 208.05 130.3) (size 0.6) (drill 0.3) (layers "F.Cu" "B.Cu") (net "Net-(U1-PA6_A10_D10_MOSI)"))
 (segment (start 205.093728 130.306272) (end 205.300001 130.306272) (width 0.2) (layer "B.Cu") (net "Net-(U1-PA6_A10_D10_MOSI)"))
 (segment (start 199.7 114.7) (end 199.7 130.7) (width 0.2) (layer "B.Cu") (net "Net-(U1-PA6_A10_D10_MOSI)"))
 (segment (start 208.05 87.35) (end 208.02 87.32) (width 0.2) (layer "B.Cu") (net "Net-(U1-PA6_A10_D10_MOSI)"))
 (segment (start 192.7 114.61) (end 199.61 114.61) (width 0.2) (layer "B.Cu") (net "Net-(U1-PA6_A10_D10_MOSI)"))
 (segment (start 199.7 130.7) (end 204.7 130.7) (width 0.2) (layer "B.Cu") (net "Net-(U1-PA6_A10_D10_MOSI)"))
 (segment (start 208.02 87.32) (end 203.95 87.32) (width 0.2) (layer "B.Cu") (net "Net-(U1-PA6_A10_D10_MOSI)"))
 (segment (start 203.87 87.4) (end 203.95 87.32) (width 0.2) (layer "B.Cu") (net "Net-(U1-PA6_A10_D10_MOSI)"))
 (segment (start 199.61 114.61) (end 199.7 114.7) (width 0.2) (layer "B.Cu") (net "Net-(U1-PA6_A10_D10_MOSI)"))
 (segment (start 204.7 130.7) (end 205.093728 130.306272) (width 0.2) (layer "B.Cu") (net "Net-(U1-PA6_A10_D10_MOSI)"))
 (segment (start 208.05 130.3) (end 208.05 87.35) (width 0.2) (layer "B.Cu") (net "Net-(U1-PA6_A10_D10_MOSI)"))
 (segment (start 206.65 131.1) (end 205.2 131.1) (width 0.2) (layer "F.Cu") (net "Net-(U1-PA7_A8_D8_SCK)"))
 (via (at 205.2 131.1) (size 0.6) (drill 0.3) (layers "F.Cu" "B.Cu") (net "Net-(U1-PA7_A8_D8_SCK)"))
 (via (at 206.65 131.1) (size 0.6) (drill 0.3) (layers "F.Cu" "B.Cu") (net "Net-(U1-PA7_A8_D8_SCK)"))
 (segment (start 180.7 131.2) (end 205.1 131.2) (width 0.2) (layer "B.Cu") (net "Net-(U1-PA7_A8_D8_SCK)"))
 (segment (start 180.61 114.61) (end 180.65 114.65) (width 0.2) (layer "B.Cu") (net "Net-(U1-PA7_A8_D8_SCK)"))
 (segment (start 180.65 114.65) (end 180.65 131.15) (width 0.2) (layer "B.Cu") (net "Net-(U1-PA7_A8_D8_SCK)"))
 (segment (start 205.1 131.2) (end 205.2 131.1) (width 0.2) (layer "B.Cu") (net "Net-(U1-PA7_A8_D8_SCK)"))
 (segment (start 206.65 131.1) (end 206.65 94.2) (width 0.2) (layer "B.Cu") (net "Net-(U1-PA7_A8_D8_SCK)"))
 (segment (start 206.65 92.4) (end 203.95 92.4) (width 0.2) (layer "B.Cu") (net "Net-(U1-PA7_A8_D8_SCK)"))
 (segment (start 201.35 92.4) (end 203.95 92.4) (width 0.2) (layer "B.Cu") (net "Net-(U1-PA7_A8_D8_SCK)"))
 (segment (start 173.65 114.61) (end 180.61 114.61) (width 0.2) (layer "B.Cu") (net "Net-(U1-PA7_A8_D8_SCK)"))
 (segment (start 206.65 94.2) (end 206.65 92.4) (width 0.2) (layer "B.Cu") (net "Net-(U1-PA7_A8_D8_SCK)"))
 (segment (start 180.65 131.15) (end 180.7 131.2) (width 0.2) (layer "B.Cu") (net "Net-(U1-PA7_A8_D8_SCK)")))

